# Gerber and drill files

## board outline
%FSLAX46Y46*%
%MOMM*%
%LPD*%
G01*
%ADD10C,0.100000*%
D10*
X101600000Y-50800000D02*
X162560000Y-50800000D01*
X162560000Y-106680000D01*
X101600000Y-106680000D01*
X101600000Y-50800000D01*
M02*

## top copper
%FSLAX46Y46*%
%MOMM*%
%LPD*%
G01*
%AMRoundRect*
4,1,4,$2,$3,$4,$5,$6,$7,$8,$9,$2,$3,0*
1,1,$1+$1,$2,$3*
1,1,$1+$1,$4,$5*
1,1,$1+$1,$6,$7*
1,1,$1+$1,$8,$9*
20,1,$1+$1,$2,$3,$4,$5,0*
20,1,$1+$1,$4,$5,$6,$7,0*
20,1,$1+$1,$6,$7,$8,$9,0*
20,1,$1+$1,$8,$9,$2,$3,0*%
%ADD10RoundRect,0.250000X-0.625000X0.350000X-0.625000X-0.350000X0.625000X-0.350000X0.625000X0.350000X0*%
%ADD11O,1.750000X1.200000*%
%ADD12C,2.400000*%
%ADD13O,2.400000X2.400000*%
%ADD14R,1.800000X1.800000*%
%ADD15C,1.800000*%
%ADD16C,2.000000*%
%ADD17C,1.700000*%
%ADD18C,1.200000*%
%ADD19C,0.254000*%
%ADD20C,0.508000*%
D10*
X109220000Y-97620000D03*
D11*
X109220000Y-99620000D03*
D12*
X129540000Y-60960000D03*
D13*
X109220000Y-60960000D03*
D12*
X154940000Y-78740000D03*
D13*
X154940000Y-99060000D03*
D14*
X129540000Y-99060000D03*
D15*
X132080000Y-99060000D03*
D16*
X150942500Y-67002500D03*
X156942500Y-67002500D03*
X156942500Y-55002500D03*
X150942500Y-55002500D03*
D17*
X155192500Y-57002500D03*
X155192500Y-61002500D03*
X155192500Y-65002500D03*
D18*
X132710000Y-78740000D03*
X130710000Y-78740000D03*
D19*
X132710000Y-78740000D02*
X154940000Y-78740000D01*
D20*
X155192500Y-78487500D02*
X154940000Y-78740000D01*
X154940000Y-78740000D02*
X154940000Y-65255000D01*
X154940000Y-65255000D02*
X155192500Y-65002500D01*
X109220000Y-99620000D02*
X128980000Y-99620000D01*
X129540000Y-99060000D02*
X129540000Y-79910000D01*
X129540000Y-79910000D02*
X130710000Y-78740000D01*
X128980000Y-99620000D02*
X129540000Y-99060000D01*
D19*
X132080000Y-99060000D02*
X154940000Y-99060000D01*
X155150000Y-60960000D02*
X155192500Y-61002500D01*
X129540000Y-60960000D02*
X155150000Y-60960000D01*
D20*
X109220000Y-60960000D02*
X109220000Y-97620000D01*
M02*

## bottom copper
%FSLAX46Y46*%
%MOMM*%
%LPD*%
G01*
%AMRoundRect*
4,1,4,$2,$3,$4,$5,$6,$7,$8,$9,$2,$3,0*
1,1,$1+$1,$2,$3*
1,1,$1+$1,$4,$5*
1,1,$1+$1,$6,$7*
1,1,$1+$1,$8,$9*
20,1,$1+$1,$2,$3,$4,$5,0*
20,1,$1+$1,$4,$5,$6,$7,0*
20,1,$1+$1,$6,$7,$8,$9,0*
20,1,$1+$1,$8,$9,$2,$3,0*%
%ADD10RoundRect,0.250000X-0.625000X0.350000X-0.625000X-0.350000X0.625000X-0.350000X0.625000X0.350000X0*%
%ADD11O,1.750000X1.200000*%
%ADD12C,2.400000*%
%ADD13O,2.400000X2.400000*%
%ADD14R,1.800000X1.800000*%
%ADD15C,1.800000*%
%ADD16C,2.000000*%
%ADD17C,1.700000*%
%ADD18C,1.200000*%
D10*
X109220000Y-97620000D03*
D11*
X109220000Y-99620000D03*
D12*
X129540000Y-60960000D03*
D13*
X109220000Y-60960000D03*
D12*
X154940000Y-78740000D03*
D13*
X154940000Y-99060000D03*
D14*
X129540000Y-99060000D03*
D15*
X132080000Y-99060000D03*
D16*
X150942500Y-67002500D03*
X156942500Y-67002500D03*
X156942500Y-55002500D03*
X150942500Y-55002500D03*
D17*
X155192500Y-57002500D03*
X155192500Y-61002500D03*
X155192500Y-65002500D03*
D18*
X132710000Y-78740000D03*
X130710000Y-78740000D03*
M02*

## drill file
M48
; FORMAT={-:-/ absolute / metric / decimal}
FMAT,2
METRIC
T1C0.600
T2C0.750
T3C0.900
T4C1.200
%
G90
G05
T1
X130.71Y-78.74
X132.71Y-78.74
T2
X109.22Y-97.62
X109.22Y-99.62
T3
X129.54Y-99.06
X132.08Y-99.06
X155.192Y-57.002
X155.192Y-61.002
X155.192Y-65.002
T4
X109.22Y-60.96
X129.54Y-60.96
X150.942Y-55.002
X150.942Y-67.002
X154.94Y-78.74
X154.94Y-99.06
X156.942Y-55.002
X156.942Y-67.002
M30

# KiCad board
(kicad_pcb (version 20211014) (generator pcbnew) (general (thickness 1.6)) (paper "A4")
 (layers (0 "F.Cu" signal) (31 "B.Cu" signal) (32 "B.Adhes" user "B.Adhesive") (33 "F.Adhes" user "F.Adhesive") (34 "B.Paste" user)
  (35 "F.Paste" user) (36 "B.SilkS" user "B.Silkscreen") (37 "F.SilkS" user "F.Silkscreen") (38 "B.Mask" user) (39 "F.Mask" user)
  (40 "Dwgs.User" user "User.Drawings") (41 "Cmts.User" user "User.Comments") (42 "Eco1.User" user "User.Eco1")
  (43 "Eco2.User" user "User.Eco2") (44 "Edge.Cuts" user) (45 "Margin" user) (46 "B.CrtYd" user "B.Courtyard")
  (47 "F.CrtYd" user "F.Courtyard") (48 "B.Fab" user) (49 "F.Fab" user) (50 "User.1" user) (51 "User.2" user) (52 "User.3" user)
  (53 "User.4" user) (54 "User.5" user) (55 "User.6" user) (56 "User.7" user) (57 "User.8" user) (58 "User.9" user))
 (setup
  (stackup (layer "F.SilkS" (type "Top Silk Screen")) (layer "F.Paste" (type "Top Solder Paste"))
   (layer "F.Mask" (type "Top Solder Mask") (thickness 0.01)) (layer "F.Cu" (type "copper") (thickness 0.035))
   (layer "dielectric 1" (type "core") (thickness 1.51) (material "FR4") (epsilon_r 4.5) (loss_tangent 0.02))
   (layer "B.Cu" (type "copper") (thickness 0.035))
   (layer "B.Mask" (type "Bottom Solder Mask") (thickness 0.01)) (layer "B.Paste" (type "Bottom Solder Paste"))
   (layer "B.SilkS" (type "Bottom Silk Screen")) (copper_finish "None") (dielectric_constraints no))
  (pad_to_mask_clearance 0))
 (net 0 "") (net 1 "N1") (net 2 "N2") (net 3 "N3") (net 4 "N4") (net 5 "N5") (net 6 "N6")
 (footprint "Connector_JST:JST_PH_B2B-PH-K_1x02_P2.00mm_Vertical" (layer "F.Cu") (at 109.22 97.62 -90)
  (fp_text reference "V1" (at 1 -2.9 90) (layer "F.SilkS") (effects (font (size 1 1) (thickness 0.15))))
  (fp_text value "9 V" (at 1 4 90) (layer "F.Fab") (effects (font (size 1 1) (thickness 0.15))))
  (pad "1" thru_hole roundrect (at 0 0 270) (size 1.2 1.75) (drill 0.75) (layers *.Cu *.Mask) (roundrect_rratio 0.208333) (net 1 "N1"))
  (pad "2" thru_hole oval (at 2 0 270) (size 1.2 1.75) (drill 0.75) (layers *.Cu *.Mask) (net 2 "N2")))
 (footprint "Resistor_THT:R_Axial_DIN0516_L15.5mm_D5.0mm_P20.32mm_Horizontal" (layer "F.Cu") (at 129.54 60.96 180)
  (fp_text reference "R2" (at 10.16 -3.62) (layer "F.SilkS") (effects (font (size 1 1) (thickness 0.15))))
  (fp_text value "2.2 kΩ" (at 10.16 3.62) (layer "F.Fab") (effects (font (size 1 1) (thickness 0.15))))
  (pad "1" thru_hole circle (at 0 0 180) (size 2.4 2.4) (drill 1.2) (layers *.Cu *.Mask) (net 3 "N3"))
  (pad "2" thru_hole oval (at 20.32 0 180) (size 2.4 2.4) (drill 1.2) (layers *.Cu *.Mask) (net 1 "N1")))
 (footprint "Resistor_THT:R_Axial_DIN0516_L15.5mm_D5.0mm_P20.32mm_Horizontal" (layer "F.Cu") (at 154.94 78.74 -90)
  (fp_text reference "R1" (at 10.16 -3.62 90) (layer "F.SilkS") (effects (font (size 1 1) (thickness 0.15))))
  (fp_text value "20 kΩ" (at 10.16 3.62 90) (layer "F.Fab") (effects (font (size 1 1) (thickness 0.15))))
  (pad "1" thru_hole circle (at 0 0 270) (size 2.4 2.4) (drill 1.2) (layers *.Cu *.Mask) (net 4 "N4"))
  (pad "2" thru_hole oval (at 20.32 0 270) (size 2.4 2.4) (drill 1.2) (layers *.Cu *.Mask) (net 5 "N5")))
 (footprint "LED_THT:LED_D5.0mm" (layer "F.Cu") (at 129.54 99.06)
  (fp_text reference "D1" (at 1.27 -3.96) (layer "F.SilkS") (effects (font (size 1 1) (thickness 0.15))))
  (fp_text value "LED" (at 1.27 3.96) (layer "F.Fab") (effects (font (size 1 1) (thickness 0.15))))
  (pad "1" thru_hole rect (at 0 0) (size 1.8 1.8) (drill 0.9) (layers *.Cu *.Mask) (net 2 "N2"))
  (pad "2" thru_hole circle (at 2.54 0) (size 1.8 1.8) (drill 0.9) (layers *.Cu *.Mask) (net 5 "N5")))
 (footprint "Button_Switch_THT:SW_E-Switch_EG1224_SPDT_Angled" (layer "F.Cu") (at 155.1925 57.0025 -90)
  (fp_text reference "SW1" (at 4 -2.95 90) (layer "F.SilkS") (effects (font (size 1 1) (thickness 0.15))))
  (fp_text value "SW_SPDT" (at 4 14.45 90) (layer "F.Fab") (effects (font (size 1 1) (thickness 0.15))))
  (pad "" thru_hole circle (at 10 4.25 270) (size 2 2) (drill 1.2) (layers *.Cu *.Mask))
  (pad "" thru_hole circle (at 10 -1.75 270) (size 2 2) (drill 1.2) (layers *.Cu *.Mask))
  (pad "" thru_hole circle (at -2 -1.75 270) (size 2 2) (drill 1.2) (layers *.Cu *.Mask))
  (pad "" thru_hole circle (at -2 4.25 270) (size 2 2) (drill 1.2) (layers *.Cu *.Mask))
  (pad "1" thru_hole circle (at 0 0 270) (size 1.7 1.7) (drill 0.9) (layers *.Cu *.Mask) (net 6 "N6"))
  (pad "2" thru_hole circle (at 4 0 270) (size 1.7 1.7) (drill 0.9) (layers *.Cu *.Mask) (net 3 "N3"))
  (pad "3" thru_hole circle (at 8 0 270) (size 1.7 1.7) (drill 0.9) (layers *.Cu *.Mask) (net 4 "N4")))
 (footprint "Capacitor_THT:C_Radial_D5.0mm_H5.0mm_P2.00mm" (layer "F.Cu") (at 132.71 78.74 180)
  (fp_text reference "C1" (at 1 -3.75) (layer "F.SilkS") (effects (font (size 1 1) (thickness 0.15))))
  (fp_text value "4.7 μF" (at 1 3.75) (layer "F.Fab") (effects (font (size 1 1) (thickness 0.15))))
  (pad "1" thru_hole circle (at 0 0 180) (size 1.2 1.2) (drill 0.6) (layers *.Cu *.Mask) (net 4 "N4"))
  (pad "2" thru_hole circle (at 2 0 180) (size 1.2 1.2) (drill 0.6) (layers *.Cu *.Mask) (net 2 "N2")))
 (gr_rect (start 101.6 50.8) (end 162.56 106.68) (layer "Edge.Cuts") (width 0.1) (fill none))
 (segment (start 132.71 78.74) (end 154.94 78.74) (width 0.254) (layer "F.Cu") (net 4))
 (segment (start 155.1925 78.4875) (end 154.94 78.74) (width 0.508) (layer "F.Cu") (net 4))
 (segment (start 154.94 78.74) (end 154.94 65.255) (width 0.508) (layer "F.Cu") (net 4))
 (segment (start 154.94 65.255) (end 155.1925 65.0025) (width 0.508) (layer "F.Cu") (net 4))
 (segment (start 109.22 99.62) (end 128.98 99.62) (width 0.508) (layer "F.Cu") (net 2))
 (segment (start 129.54 99.06) (end 129.54 79.91) (width 0.508) (layer "F.Cu") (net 2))
 (segment (start 129.54 79.91) (end 130.71 78.74) (width 0.508) (layer "F.Cu") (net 2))
 (segment (start 128.98 99.62) (end 129.54 99.06) (width 0.508) (layer "F.Cu") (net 2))
 (segment (start 132.08 99.06) (end 154.94 99.06) (width 0.254) (layer "F.Cu") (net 5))
 (segment (start 155.15 60.96) (end 155.1925 61.0025) (width 0.254) (layer "F.Cu") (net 3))
 (segment (start 129.54 60.96) (end 155.15 60.96) (width 0.254) (layer "F.Cu") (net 3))
 (segment (start 109.22 60.96) (end 109.22 97.62) (width 0.508) (layer "F.Cu") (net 1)))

